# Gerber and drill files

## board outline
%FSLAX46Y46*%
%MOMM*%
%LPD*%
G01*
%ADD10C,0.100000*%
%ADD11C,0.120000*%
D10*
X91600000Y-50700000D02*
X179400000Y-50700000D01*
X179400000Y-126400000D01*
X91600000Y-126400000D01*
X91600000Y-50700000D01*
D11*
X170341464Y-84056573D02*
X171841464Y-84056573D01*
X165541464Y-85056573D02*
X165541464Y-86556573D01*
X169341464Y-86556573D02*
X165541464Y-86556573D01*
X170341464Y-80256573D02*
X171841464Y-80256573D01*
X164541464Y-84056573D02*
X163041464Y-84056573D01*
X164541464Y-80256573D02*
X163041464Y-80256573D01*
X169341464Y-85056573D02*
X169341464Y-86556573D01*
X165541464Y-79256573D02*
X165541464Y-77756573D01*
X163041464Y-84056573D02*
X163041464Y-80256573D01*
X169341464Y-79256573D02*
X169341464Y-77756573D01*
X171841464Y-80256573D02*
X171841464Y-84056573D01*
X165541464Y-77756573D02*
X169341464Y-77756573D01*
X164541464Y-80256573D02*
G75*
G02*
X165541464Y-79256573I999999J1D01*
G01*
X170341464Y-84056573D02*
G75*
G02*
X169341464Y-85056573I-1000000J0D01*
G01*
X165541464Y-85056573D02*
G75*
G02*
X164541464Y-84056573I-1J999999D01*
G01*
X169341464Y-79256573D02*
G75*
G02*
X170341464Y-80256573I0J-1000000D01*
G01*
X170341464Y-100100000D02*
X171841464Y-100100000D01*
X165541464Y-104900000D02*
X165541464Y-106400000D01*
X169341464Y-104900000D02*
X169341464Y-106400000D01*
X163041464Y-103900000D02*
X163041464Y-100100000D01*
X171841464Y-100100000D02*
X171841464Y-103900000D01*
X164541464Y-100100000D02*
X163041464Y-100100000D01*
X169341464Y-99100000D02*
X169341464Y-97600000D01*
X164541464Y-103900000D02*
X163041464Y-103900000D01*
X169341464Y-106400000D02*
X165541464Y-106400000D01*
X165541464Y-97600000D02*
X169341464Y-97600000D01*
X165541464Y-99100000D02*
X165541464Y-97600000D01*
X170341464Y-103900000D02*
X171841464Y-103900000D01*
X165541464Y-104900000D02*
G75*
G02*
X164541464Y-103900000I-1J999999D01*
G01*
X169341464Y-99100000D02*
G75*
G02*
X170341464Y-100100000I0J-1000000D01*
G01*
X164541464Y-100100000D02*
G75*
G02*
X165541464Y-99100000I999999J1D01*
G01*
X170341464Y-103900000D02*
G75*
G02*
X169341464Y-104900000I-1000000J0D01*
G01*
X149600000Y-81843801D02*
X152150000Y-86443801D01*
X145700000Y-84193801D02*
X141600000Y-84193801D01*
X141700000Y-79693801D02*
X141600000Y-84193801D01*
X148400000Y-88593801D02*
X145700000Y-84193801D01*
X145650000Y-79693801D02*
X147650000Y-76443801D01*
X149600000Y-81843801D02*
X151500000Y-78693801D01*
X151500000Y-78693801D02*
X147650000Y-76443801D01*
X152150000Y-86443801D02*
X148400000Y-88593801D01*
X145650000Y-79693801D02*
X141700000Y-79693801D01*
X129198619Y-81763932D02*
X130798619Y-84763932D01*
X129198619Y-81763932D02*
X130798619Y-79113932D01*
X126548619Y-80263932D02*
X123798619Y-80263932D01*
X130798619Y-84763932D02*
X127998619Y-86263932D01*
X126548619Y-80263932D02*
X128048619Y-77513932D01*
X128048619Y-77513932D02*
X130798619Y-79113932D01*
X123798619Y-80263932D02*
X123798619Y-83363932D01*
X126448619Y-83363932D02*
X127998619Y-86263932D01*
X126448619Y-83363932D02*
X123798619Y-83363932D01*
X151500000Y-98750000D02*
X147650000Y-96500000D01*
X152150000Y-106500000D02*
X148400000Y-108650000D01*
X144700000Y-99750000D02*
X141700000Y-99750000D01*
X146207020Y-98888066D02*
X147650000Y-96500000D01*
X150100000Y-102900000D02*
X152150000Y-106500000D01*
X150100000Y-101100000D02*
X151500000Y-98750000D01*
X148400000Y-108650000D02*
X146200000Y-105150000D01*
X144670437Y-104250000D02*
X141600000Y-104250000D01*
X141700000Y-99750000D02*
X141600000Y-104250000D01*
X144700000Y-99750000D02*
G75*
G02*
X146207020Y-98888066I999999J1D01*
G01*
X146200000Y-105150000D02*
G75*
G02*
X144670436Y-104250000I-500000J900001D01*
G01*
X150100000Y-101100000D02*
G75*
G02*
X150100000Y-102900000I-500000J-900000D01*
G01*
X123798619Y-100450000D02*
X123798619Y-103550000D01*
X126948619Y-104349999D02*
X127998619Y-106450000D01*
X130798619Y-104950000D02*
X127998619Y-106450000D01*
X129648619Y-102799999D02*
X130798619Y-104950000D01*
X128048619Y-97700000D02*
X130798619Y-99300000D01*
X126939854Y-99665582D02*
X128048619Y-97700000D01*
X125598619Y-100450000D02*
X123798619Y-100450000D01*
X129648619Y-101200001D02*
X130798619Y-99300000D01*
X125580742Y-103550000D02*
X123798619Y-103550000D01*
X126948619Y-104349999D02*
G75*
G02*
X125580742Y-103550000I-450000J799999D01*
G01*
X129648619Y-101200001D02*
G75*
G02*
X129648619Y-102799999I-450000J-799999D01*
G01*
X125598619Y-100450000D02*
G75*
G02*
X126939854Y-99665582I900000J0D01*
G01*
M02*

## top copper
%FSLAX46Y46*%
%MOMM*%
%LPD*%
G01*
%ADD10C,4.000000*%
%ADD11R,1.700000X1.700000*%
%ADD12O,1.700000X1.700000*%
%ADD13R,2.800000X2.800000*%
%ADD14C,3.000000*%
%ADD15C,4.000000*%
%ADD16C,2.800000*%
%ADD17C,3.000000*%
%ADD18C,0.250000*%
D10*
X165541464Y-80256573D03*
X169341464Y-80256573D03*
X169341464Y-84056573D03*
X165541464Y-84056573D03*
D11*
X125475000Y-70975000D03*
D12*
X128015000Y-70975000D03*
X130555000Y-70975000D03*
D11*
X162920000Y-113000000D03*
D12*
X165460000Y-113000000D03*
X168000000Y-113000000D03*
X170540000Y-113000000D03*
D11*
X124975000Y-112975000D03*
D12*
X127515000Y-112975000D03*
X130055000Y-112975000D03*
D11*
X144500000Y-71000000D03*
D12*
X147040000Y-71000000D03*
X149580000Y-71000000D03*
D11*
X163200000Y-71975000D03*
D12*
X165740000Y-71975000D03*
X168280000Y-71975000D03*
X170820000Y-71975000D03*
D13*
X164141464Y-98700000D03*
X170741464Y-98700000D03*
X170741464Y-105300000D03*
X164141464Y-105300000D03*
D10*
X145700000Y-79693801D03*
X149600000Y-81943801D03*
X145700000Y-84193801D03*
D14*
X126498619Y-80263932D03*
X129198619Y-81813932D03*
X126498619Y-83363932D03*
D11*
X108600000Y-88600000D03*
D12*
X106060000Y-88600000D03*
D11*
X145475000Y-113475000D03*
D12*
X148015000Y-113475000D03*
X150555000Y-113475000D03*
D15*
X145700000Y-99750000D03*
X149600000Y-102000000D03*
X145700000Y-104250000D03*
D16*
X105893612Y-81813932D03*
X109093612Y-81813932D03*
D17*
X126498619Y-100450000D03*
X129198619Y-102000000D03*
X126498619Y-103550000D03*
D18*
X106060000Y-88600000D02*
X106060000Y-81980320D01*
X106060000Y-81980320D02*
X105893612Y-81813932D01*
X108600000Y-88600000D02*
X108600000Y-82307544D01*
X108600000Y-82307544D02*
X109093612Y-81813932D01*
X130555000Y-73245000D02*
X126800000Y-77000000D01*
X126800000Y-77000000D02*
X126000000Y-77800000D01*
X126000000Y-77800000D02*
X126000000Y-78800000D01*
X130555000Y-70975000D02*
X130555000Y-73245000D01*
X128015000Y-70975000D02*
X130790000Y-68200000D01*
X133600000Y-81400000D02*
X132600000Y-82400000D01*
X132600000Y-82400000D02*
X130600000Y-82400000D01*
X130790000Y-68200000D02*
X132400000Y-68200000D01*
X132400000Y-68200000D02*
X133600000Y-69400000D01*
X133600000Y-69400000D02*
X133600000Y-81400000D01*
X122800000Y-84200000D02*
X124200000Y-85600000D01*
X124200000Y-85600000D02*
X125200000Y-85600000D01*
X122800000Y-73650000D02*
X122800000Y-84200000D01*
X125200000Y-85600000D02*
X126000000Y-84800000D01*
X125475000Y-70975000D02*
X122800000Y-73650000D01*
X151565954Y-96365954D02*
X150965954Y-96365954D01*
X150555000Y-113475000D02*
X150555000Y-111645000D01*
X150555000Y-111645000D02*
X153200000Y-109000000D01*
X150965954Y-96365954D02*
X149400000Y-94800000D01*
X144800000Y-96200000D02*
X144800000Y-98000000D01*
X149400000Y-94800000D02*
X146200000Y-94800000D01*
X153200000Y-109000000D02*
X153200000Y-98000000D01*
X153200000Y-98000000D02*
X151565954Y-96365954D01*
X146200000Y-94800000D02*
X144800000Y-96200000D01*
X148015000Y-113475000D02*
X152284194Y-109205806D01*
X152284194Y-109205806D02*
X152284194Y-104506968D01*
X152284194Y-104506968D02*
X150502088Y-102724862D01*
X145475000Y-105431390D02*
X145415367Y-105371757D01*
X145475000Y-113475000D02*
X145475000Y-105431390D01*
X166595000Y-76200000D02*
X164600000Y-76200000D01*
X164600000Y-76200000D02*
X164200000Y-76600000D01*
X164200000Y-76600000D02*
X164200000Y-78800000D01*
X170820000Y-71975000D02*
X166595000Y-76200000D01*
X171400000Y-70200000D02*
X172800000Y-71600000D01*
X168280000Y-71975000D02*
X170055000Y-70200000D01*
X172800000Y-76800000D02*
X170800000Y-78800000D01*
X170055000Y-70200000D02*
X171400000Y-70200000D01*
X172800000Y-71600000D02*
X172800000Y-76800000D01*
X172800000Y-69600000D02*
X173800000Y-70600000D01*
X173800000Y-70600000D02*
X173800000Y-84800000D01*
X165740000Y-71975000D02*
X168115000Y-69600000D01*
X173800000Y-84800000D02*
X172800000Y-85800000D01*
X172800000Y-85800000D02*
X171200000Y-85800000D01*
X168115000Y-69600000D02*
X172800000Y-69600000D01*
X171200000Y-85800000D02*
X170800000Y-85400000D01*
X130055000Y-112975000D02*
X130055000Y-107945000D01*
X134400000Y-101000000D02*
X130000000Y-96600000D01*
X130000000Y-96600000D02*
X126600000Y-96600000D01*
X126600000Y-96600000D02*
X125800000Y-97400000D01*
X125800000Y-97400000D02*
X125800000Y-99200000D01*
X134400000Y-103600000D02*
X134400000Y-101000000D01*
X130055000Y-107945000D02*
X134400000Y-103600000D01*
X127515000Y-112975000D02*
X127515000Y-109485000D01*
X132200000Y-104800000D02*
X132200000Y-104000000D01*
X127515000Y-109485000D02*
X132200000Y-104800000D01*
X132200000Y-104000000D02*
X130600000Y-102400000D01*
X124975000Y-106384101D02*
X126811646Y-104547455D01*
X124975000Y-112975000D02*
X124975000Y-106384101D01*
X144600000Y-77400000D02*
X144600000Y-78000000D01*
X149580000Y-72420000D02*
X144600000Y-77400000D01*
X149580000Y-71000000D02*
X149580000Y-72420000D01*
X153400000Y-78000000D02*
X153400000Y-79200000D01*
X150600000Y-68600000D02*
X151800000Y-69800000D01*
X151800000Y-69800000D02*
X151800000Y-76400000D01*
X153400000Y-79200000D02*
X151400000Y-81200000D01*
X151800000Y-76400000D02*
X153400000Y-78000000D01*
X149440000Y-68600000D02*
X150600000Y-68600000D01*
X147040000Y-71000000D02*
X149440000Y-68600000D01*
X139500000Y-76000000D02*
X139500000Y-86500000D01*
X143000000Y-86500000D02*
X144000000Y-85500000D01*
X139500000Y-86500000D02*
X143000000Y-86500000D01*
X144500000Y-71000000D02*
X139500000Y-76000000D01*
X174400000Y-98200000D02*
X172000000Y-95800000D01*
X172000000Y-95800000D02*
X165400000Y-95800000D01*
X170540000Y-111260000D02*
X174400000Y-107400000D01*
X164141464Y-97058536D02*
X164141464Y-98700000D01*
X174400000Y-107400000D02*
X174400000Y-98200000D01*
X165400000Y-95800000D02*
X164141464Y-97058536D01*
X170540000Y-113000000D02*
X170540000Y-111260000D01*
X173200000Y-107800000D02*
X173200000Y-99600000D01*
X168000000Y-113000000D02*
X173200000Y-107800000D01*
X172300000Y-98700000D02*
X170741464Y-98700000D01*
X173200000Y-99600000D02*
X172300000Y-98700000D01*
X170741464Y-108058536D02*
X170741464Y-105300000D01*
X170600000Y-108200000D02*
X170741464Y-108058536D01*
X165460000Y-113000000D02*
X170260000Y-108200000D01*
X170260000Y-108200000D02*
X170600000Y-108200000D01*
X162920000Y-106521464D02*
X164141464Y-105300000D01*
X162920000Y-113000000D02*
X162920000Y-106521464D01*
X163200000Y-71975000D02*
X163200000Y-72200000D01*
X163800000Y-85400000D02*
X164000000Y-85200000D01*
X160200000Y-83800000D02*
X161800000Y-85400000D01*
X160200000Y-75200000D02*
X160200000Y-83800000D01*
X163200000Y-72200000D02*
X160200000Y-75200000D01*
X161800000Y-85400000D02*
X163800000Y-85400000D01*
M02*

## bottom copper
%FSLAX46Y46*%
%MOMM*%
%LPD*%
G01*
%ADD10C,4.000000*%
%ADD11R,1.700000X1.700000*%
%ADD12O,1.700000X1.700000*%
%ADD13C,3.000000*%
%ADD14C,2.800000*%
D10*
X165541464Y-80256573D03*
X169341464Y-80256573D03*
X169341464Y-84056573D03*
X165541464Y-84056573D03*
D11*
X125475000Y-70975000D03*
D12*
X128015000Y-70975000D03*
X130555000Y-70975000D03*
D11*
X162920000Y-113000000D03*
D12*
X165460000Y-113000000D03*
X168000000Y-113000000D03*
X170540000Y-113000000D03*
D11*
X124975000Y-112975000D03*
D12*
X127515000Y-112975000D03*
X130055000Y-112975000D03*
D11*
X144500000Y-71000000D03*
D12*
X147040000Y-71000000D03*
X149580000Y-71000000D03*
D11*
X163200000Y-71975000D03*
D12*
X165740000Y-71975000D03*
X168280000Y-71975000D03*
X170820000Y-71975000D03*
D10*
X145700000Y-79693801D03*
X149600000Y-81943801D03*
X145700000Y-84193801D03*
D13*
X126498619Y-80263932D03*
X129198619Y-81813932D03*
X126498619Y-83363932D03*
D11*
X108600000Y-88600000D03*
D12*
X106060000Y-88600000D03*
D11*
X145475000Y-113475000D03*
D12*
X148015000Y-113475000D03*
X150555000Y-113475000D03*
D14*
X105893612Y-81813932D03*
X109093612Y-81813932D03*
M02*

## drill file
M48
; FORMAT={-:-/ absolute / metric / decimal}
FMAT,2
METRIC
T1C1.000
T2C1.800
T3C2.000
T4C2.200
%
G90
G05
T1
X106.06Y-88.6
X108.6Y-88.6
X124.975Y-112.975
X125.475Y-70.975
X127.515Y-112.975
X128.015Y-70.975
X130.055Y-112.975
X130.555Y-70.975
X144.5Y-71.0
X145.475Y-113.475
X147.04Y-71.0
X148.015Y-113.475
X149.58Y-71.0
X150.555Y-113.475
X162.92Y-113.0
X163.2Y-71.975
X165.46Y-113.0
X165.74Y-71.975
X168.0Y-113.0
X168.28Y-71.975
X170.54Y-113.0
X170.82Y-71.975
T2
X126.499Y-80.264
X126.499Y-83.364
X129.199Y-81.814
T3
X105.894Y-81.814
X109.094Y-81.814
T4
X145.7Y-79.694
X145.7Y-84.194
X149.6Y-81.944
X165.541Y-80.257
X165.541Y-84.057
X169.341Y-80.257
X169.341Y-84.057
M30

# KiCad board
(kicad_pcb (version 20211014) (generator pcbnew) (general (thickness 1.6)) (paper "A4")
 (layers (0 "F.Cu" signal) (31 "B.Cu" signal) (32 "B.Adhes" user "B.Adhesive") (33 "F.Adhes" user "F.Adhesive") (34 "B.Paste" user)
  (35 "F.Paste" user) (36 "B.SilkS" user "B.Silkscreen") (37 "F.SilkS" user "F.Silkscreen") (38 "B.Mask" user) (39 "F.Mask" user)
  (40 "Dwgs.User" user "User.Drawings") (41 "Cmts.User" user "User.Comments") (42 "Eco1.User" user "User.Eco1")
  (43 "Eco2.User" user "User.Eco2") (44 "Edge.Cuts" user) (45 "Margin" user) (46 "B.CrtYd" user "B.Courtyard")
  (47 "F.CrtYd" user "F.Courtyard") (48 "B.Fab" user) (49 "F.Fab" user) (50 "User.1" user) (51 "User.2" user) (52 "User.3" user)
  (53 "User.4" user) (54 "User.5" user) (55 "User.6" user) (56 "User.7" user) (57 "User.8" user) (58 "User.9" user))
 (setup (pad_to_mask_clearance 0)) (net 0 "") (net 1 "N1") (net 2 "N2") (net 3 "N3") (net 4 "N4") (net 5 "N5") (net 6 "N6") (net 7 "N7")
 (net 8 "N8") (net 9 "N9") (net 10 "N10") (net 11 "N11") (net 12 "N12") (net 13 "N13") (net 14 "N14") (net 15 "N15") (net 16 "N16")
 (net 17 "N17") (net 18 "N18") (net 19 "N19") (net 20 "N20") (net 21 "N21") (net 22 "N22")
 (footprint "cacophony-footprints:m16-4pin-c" (layer "F.Cu") (at 167.441464 82.156573)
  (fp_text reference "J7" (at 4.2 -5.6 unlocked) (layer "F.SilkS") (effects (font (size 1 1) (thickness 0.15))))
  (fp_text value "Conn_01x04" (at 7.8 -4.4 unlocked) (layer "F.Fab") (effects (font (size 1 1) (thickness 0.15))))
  (fp_line (start 2.9 1.9) (end 4.4 1.9) (layer "Edge.Cuts") (width 0.12))
  (fp_line (start -1.9 2.9) (end -1.9 4.4) (layer "Edge.Cuts") (width 0.12))
  (fp_line (start 1.9 4.4) (end -1.9 4.4) (layer "Edge.Cuts") (width 0.12))
  (fp_line (start 2.9 -1.9) (end 4.4 -1.9) (layer "Edge.Cuts") (width 0.12))
  (fp_line (start -2.9 1.9) (end -4.4 1.9) (layer "Edge.Cuts") (width 0.12))
  (fp_line (start -2.9 -1.9) (end -4.4 -1.9) (layer "Edge.Cuts") (width 0.12))
  (fp_line (start 1.9 2.9) (end 1.9 4.4) (layer "Edge.Cuts") (width 0.12))
  (fp_line (start -1.9 -2.9) (end -1.9 -4.4) (layer "Edge.Cuts") (width 0.12))
  (fp_line (start -4.4 1.9) (end -4.4 -1.9) (layer "Edge.Cuts") (width 0.12))
  (fp_line (start 1.9 -2.9) (end 1.9 -4.4) (layer "Edge.Cuts") (width 0.12))
  (fp_line (start 4.4 -1.9) (end 4.4 1.9) (layer "Edge.Cuts") (width 0.12))
  (fp_line (start -1.9 -4.4) (end 1.9 -4.4) (layer "Edge.Cuts") (width 0.12))
  (fp_arc (start -2.9 -1.9) (mid -2.607107 -2.607107) (end -1.9 -2.9) (layer "Edge.Cuts") (width 0.12))
  (fp_arc (start 2.9 1.9) (mid 2.607107 2.607107) (end 1.9 2.9) (layer "Edge.Cuts") (width 0.12))
  (fp_arc (start -1.9 2.9) (mid -2.607107 2.607107) (end -2.9 1.9) (layer "Edge.Cuts") (width 0.12))
  (fp_arc (start 1.9 -2.9) (mid 2.607107 -2.607107) (end 2.9 -1.9) (layer "Edge.Cuts") (width 0.12))
  (pad "1" thru_hole circle (at -1.9 -1.9) (size 4 4) (drill 2.2) (layers *.Cu *.Mask) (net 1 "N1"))
  (pad "2" thru_hole circle (at 1.9 -1.9) (size 4 4) (drill 2.2) (layers *.Cu *.Mask) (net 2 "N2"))
  (pad "3" thru_hole circle (at 1.9 1.9) (size 4 4) (drill 2.2) (layers *.Cu *.Mask) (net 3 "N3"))
  (pad "4" thru_hole circle (at -1.9 1.9) (size 4 4) (drill 2.2) (layers *.Cu *.Mask) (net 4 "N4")))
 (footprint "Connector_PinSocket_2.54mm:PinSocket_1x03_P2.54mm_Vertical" (layer "F.Cu") (at 125.475 70.975 90)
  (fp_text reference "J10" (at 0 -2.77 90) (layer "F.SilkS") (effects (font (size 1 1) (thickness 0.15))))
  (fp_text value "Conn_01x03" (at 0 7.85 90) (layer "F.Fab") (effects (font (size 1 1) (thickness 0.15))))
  (pad "1" thru_hole rect (at 0 0 90) (size 1.7 1.7) (drill 1) (layers *.Cu *.Mask) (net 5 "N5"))
  (pad "2" thru_hole oval (at 0 2.54 90) (size 1.7 1.7) (drill 1) (layers *.Cu *.Mask) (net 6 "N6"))
  (pad "3" thru_hole oval (at 0 5.08 90) (size 1.7 1.7) (drill 1) (layers *.Cu *.Mask) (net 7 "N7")))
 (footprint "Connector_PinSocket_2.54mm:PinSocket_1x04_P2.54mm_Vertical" (layer "F.Cu") (at 162.92 113 90)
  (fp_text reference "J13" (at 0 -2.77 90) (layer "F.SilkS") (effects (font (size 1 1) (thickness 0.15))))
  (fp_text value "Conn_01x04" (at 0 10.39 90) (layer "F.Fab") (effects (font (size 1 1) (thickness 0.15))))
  (pad "1" thru_hole rect (at 0 0 90) (size 1.7 1.7) (drill 1) (layers *.Cu *.Mask) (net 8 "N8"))
  (pad "2" thru_hole oval (at 0 2.54 90) (size 1.7 1.7) (drill 1) (layers *.Cu *.Mask) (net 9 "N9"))
  (pad "3" thru_hole oval (at 0 5.08 90) (size 1.7 1.7) (drill 1) (layers *.Cu *.Mask) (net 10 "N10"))
  (pad "4" thru_hole oval (at 0 7.62 90) (size 1.7 1.7) (drill 1) (layers *.Cu *.Mask) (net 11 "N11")))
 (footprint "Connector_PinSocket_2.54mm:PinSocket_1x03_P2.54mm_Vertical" (layer "F.Cu") (at 124.975 112.975 90)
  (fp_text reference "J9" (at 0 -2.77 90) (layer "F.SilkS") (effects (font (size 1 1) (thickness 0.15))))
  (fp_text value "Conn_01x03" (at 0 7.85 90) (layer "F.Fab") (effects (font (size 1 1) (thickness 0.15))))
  (pad "1" thru_hole rect (at 0 0 90) (size 1.7 1.7) (drill 1) (layers *.Cu *.Mask) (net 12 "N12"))
  (pad "2" thru_hole oval (at 0 2.54 90) (size 1.7 1.7) (drill 1) (layers *.Cu *.Mask) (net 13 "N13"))
  (pad "3" thru_hole oval (at 0 5.08 90) (size 1.7 1.7) (drill 1) (layers *.Cu *.Mask) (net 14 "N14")))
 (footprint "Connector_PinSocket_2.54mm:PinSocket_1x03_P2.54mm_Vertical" (layer "F.Cu") (at 144.5 71 90)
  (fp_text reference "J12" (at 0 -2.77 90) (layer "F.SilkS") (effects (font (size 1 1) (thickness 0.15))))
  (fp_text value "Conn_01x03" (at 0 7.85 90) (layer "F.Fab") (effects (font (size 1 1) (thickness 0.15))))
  (pad "1" thru_hole rect (at 0 0 90) (size 1.7 1.7) (drill 1) (layers *.Cu *.Mask) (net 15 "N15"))
  (pad "2" thru_hole oval (at 0 2.54 90) (size 1.7 1.7) (drill 1) (layers *.Cu *.Mask) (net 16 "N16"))
  (pad "3" thru_hole oval (at 0 5.08 90) (size 1.7 1.7) (drill 1) (layers *.Cu *.Mask) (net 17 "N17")))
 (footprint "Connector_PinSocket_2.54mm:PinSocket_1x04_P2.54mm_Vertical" (layer "F.Cu") (at 163.2 71.975 90)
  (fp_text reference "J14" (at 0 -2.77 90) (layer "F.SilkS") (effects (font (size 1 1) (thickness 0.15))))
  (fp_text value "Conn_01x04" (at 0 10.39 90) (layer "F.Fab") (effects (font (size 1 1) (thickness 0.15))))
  (pad "1" thru_hole rect (at 0 0 90) (size 1.7 1.7) (drill 1) (layers *.Cu *.Mask) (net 4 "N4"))
  (pad "2" thru_hole oval (at 0 2.54 90) (size 1.7 1.7) (drill 1) (layers *.Cu *.Mask) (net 3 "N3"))
  (pad "3" thru_hole oval (at 0 5.08 90) (size 1.7 1.7) (drill 1) (layers *.Cu *.Mask) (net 2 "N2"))
  (pad "4" thru_hole oval (at 0 7.62 90) (size 1.7 1.7) (drill 1) (layers *.Cu *.Mask) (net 1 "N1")))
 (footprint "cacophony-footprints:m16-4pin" (layer "F.Cu") (at 167.441464 102)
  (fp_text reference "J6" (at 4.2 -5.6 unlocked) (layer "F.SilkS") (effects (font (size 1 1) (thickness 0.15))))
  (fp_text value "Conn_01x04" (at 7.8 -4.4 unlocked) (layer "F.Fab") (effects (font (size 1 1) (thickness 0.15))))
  (fp_line (start 2.9 -1.9) (end 4.4 -1.9) (layer "Edge.Cuts") (width 0.12))
  (fp_line (start -1.9 2.9) (end -1.9 4.4) (layer "Edge.Cuts") (width 0.12))
  (fp_line (start 1.9 2.9) (end 1.9 4.4) (layer "Edge.Cuts") (width 0.12))
  (fp_line (start -4.4 1.9) (end -4.4 -1.9) (layer "Edge.Cuts") (width 0.12))
  (fp_line (start 4.4 -1.9) (end 4.4 1.9) (layer "Edge.Cuts") (width 0.12))
  (fp_line (start -2.9 -1.9) (end -4.4 -1.9) (layer "Edge.Cuts") (width 0.12))
  (fp_line (start 1.9 -2.9) (end 1.9 -4.4) (layer "Edge.Cuts") (width 0.12))
  (fp_line (start -2.9 1.9) (end -4.4 1.9) (layer "Edge.Cuts") (width 0.12))
  (fp_line (start 1.9 4.4) (end -1.9 4.4) (layer "Edge.Cuts") (width 0.12))
  (fp_line (start -1.9 -4.4) (end 1.9 -4.4) (layer "Edge.Cuts") (width 0.12))
  (fp_line (start -1.9 -2.9) (end -1.9 -4.4) (layer "Edge.Cuts") (width 0.12))
  (fp_line (start 2.9 1.9) (end 4.4 1.9) (layer "Edge.Cuts") (width 0.12))
  (fp_arc (start -1.9 2.9) (mid -2.607107 2.607107) (end -2.9 1.9) (layer "Edge.Cuts") (width 0.12))
  (fp_arc (start 1.9 -2.9) (mid 2.607107 -2.607107) (end 2.9 -1.9) (layer "Edge.Cuts") (width 0.12))
  (fp_arc (start -2.9 -1.9) (mid -2.607107 -2.607107) (end -1.9 -2.9) (layer "Edge.Cuts") (width 0.12))
  (fp_arc (start 2.9 1.9) (mid 2.607107 2.607107) (end 1.9 2.9) (layer "Edge.Cuts") (width 0.12))
  (pad "1" smd rect (at -3.3 -3.3) (size 2.8 2.8) (layers "F.Cu" "F.Paste" "F.Mask") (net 11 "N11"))
  (pad "2" smd rect (at 3.3 -3.3) (size 2.8 2.8) (layers "F.Cu" "F.Paste" "F.Mask") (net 10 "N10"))
  (pad "3" smd rect (at 3.3 3.3) (size 2.8 2.8) (layers "F.Cu" "F.Paste" "F.Mask") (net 9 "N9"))
  (pad "4" smd rect (at -3.3 3.3) (size 2.8 2.8) (layers "F.Cu" "F.Paste" "F.Mask") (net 8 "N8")))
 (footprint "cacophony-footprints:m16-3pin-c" (layer "F.Cu") (at 147 81.943801)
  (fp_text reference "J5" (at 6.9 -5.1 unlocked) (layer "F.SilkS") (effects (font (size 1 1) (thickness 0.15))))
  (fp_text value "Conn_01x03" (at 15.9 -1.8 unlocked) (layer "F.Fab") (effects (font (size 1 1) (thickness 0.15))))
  (fp_line (start 2.6 -0.1) (end 5.15 4.5) (layer "Edge.Cuts") (width 0.12))
  (fp_line (start -1.3 2.25) (end -5.4 2.25) (layer "Edge.Cuts") (width 0.12))
  (fp_line (start -5.3 -2.25) (end -5.4 2.25) (layer "Edge.Cuts") (width 0.12))
  (fp_line (start 1.4 6.65) (end -1.3 2.25) (layer "Edge.Cuts") (width 0.12))
  (fp_line (start -1.35 -2.25) (end 0.65 -5.5) (layer "Edge.Cuts") (width 0.12))
  (fp_line (start 2.6 -0.1) (end 4.5 -3.25) (layer "Edge.Cuts") (width 0.12))
  (fp_line (start 4.5 -3.25) (end 0.65 -5.5) (layer "Edge.Cuts") (width 0.12))
  (fp_line (start 5.15 4.5) (end 1.4 6.65) (layer "Edge.Cuts") (width 0.12))
  (fp_line (start -1.35 -2.25) (end -5.3 -2.25) (layer "Edge.Cuts") (width 0.12))
  (pad "1" thru_hole circle (at -1.3 -2.25) (size 4 4) (drill 2.2) (layers *.Cu *.Mask) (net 17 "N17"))
  (pad "2" thru_hole circle (at 2.6 0) (size 4 4) (drill 2.2) (layers *.Cu *.Mask) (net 16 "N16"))
  (pad "3" thru_hole circle (at -1.3 2.25) (size 4 4) (drill 2.2) (layers *.Cu *.Mask) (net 15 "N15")))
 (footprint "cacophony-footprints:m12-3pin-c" (layer "F.Cu") (at 127.398619 81.813932)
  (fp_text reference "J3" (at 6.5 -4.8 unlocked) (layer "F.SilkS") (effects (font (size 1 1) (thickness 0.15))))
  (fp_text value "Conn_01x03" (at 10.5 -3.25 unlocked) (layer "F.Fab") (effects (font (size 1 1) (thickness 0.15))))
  (fp_line (start 1.8 -0.05) (end 3.4 2.95) (layer "Edge.Cuts") (width 0.12))
  (fp_line (start 1.8 -0.05) (end 3.4 -2.7) (layer "Edge.Cuts") (width 0.12))
  (fp_line (start -0.85 -1.55) (end -3.6 -1.55) (layer "Edge.Cuts") (width 0.12))
  (fp_line (start 3.4 2.95) (end 0.6 4.45) (layer "Edge.Cuts") (width 0.12))
  (fp_line (start -0.85 -1.55) (end 0.65 -4.3) (layer "Edge.Cuts") (width 0.12))
  (fp_line (start 0.65 -4.3) (end 3.4 -2.7) (layer "Edge.Cuts") (width 0.12))
  (fp_line (start -3.6 -1.55) (end -3.6 1.55) (layer "Edge.Cuts") (width 0.12))
  (fp_line (start -0.95 1.55) (end 0.6 4.45) (layer "Edge.Cuts") (width 0.12))
  (fp_line (start -0.95 1.55) (end -3.6 1.55) (layer "Edge.Cuts") (width 0.12))
  (pad "1" thru_hole circle (at -0.9 -1.55) (size 3 3) (drill 1.8) (layers *.Cu *.Mask) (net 7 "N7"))
  (pad "2" thru_hole circle (at 1.8 0) (size 3 3) (drill 1.8) (layers *.Cu *.Mask) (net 6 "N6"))
  (pad "3" thru_hole circle (at -0.9 1.55) (size 3 3) (drill 1.8) (layers *.Cu *.Mask) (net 5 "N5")))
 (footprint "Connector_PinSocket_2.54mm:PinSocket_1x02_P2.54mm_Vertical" (layer "F.Cu") (at 108.6 88.6 -90)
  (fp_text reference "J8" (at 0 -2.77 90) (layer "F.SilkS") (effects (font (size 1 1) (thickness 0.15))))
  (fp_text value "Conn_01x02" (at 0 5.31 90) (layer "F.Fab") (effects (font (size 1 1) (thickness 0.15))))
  (pad "1" thru_hole rect (at 0 0 270) (size 1.7 1.7) (drill 1) (layers *.Cu *.Mask) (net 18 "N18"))
  (pad "2" thru_hole oval (at 0 2.54 270) (size 1.7 1.7) (drill 1) (layers *.Cu *.Mask) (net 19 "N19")))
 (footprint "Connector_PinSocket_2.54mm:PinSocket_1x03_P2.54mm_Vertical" (layer "F.Cu") (at 145.475 113.475 90)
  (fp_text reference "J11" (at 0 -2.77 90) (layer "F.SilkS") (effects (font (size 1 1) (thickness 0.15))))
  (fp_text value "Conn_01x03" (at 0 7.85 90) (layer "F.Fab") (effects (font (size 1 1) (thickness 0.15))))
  (pad "1" thru_hole rect (at 0 0 90) (size 1.7 1.7) (drill 1) (layers *.Cu *.Mask) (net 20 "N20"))
  (pad "2" thru_hole oval (at 0 2.54 90) (size 1.7 1.7) (drill 1) (layers *.Cu *.Mask) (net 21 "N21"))
  (pad "3" thru_hole oval (at 0 5.08 90) (size 1.7 1.7) (drill 1) (layers *.Cu *.Mask) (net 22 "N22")))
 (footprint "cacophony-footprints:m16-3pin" (layer "F.Cu") (at 147 102)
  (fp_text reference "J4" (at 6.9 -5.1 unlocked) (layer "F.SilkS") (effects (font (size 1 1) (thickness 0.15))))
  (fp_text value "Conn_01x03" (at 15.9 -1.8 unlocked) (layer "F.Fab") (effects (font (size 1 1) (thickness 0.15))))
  (fp_line (start 4.5 -3.25) (end 0.65 -5.5) (layer "Edge.Cuts") (width 0.12))
  (fp_line (start 5.15 4.5) (end 1.4 6.65) (layer "Edge.Cuts") (width 0.12))
  (fp_line (start -2.3 -2.25) (end -5.3 -2.25) (layer "Edge.Cuts") (width 0.12))
  (fp_line (start -0.79298 -3.111934) (end 0.65 -5.5) (layer "Edge.Cuts") (width 0.12))
  (fp_line (start 3.1 0.9) (end 5.15 4.5) (layer "Edge.Cuts") (width 0.12))
  (fp_line (start 3.1 -0.9) (end 4.5 -3.25) (layer "Edge.Cuts") (width 0.12))
  (fp_line (start 1.4 6.65) (end -0.8 3.15) (layer "Edge.Cuts") (width 0.12))
  (fp_line (start -2.329563 2.25) (end -5.4 2.25) (layer "Edge.Cuts") (width 0.12))
  (fp_line (start -5.3 -2.25) (end -5.4 2.25) (layer "Edge.Cuts") (width 0.12))
  (fp_arc (start -2.3 -2.25) (mid -1.796478 -3.11805) (end -0.79298 -3.111934) (layer "Edge.Cuts") (width 0.12))
  (fp_arc (start -0.8 3.15) (mid -1.82212 3.13735) (end -2.329563 2.25) (layer "Edge.Cuts") (width 0.12))
  (fp_arc (start 3.1 -0.9) (mid 3.629563 0) (end 3.1 0.9) (layer "Edge.Cuts") (width 0.12))
  (pad "1" smd circle (at -1.3 -2.25) (size 4 4) (layers "F.Cu" "F.Paste" "F.Mask") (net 22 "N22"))
  (pad "2" smd circle (at 2.6 0) (size 4 4) (layers "F.Cu" "F.Paste" "F.Mask") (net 21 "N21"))
  (pad "3" smd circle (at -1.3 2.25) (size 4 4) (layers "F.Cu" "F.Paste" "F.Mask") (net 20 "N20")))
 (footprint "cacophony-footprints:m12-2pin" (layer "F.Cu") (at 107.493612 81.813932)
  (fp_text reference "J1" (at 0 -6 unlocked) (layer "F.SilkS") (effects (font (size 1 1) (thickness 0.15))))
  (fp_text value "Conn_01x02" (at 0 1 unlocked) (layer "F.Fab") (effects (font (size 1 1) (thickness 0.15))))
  (pad "1" thru_hole circle (at -1.6 0) (size 2.8 2.8) (drill 2) (layers *.Cu *.Mask) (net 19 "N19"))
  (pad "2" thru_hole circle (at 1.6 0) (size 2.8 2.8) (drill 2) (layers *.Cu *.Mask) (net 18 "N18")))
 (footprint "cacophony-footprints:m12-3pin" (layer "F.Cu") (at 127.398619 102)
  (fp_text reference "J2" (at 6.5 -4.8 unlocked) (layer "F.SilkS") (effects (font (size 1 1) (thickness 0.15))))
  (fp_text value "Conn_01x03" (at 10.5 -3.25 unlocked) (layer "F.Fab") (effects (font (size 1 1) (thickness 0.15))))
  (fp_line (start -3.6 -1.55) (end -3.6 1.55) (layer "Edge.Cuts") (width 0.12))
  (fp_line (start -0.45 2.349999) (end 0.6 4.45) (layer "Edge.Cuts") (width 0.12))
  (fp_line (start 3.4 2.95) (end 0.6 4.45) (layer "Edge.Cuts") (width 0.12))
  (fp_line (start 2.25 0.799999) (end 3.4 2.95) (layer "Edge.Cuts") (width 0.12))
  (fp_line (start 0.65 -4.3) (end 3.4 -2.7) (layer "Edge.Cuts") (width 0.12))
  (fp_line (start -0.458765 -2.334418) (end 0.65 -4.3) (layer "Edge.Cuts") (width 0.12))
  (fp_line (start -1.8 -1.55) (end -3.6 -1.55) (layer "Edge.Cuts") (width 0.12))
  (fp_line (start 2.25 -0.799999) (end 3.4 -2.7) (layer "Edge.Cuts") (width 0.12))
  (fp_line (start -1.817877 1.55) (end -3.6 1.55) (layer "Edge.Cuts") (width 0.12))
  (fp_arc (start -0.45 2.349999) (mid -1.363387 2.34232) (end -1.817877 1.55) (layer "Edge.Cuts") (width 0.12))
  (fp_arc (start 2.25 -0.799999) (mid 2.717877 0) (end 2.25 0.799999) (layer "Edge.Cuts") (width 0.12))
  (fp_arc (start -1.8 -1.55) (mid -1.354361 -2.326889) (end -0.458765 -2.334418) (layer "Edge.Cuts") (width 0.12))
  (pad "1" smd circle (at -0.9 -1.55) (size 3 3) (layers "F.Cu" "F.Paste" "F.Mask") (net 14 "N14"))
  (pad "2" smd circle (at 1.8 0) (size 3 3) (layers "F.Cu" "F.Paste" "F.Mask") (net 13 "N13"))
  (pad "3" smd circle (at -0.9 1.55) (size 3 3) (layers "F.Cu" "F.Paste" "F.Mask") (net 12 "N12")))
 (gr_rect (start 91.6 50.7) (end 179.4 126.4) (layer "Edge.Cuts") (width 0.1) (fill none))
 (segment (start 106.06 88.6) (end 106.06 81.98032) (width 0.25) (layer "F.Cu") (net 19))
 (segment (start 106.06 81.98032) (end 105.893612 81.813932) (width 0.25) (layer "F.Cu") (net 19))
 (segment (start 108.6 88.6) (end 108.6 82.307544) (width 0.25) (layer "F.Cu") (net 18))
 (segment (start 108.6 82.307544) (end 109.093612 81.813932) (width 0.25) (layer "F.Cu") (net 18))
 (segment (start 130.555 73.245) (end 126.8 77) (width 0.25) (layer "F.Cu") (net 7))
 (segment (start 126.8 77) (end 126 77.8) (width 0.25) (layer "F.Cu") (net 7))
 (segment (start 126 77.8) (end 126 78.8) (width 0.25) (layer "F.Cu") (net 7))
 (segment (start 130.555 70.975) (end 130.555 73.245) (width 0.25) (layer "F.Cu") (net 7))
 (segment (start 128.015 70.975) (end 130.79 68.2) (width 0.25) (layer "F.Cu") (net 6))
 (segment (start 133.6 81.4) (end 132.6 82.4) (width 0.25) (layer "F.Cu") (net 6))
 (segment (start 132.6 82.4) (end 130.6 82.4) (width 0.25) (layer "F.Cu") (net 6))
 (segment (start 130.79 68.2) (end 132.4 68.2) (width 0.25) (layer "F.Cu") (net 6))
 (segment (start 132.4 68.2) (end 133.6 69.4) (width 0.25) (layer "F.Cu") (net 6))
 (segment (start 133.6 69.4) (end 133.6 81.4) (width 0.25) (layer "F.Cu") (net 6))
 (segment (start 122.8 84.2) (end 124.2 85.6) (width 0.25) (layer "F.Cu") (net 5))
 (segment (start 124.2 85.6) (end 125.2 85.6) (width 0.25) (layer "F.Cu") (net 5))
 (segment (start 122.8 73.65) (end 122.8 84.2) (width 0.25) (layer "F.Cu") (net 5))
 (segment (start 125.2 85.6) (end 126 84.8) (width 0.25) (layer "F.Cu") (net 5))
 (segment (start 125.475 70.975) (end 122.8 73.65) (width 0.25) (layer "F.Cu") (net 5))
 (segment (start 151.565954 96.365954) (end 150.965954 96.365954) (width 0.25) (layer "F.Cu") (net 22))
 (segment (start 150.555 113.475) (end 150.555 111.645) (width 0.25) (layer "F.Cu") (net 22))
 (segment (start 150.555 111.645) (end 153.2 109) (width 0.25) (layer "F.Cu") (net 22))
 (segment (start 150.965954 96.365954) (end 149.4 94.8) (width 0.25) (layer "F.Cu") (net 22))
 (segment (start 144.8 96.2) (end 144.8 98) (width 0.25) (layer "F.Cu") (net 22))
 (segment (start 149.4 94.8) (end 146.2 94.8) (width 0.25) (layer "F.Cu") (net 22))
 (segment (start 153.2 109) (end 153.2 98) (width 0.25) (layer "F.Cu") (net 22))
 (segment (start 153.2 98) (end 151.565954 96.365954) (width 0.25) (layer "F.Cu") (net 22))
 (segment (start 146.2 94.8) (end 144.8 96.2) (width 0.25) (layer "F.Cu") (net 22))
 (segment (start 148.015 113.475) (end 152.284194 109.205806) (width 0.25) (layer "F.Cu") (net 21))
 (segment (start 152.284194 109.205806) (end 152.284194 104.506968) (width 0.25) (layer "F.Cu") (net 21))
 (segment (start 152.284194 104.506968) (end 150.502088 102.724862) (width 0.25) (layer "F.Cu") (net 21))
 (segment (start 145.475 105.43139) (end 145.415367 105.371757) (width 0.25) (layer "F.Cu") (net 20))
 (segment (start 145.475 113.475) (end 145.475 105.43139) (width 0.25) (layer "F.Cu") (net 20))
 (segment (start 166.595 76.2) (end 164.6 76.2) (width 0.25) (layer "F.Cu") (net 1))
 (segment (start 164.6 76.2) (end 164.2 76.6) (width 0.25) (layer "F.Cu") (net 1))
 (segment (start 164.2 76.6) (end 164.2 78.8) (width 0.25) (layer "F.Cu") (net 1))
 (segment (start 170.82 71.975) (end 166.595 76.2) (width 0.25) (layer "F.Cu") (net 1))
 (segment (start 171.4 70.2) (end 172.8 71.6) (width 0.25) (layer "F.Cu") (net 2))
 (segment (start 168.28 71.975) (end 170.055 70.2) (width 0.25) (layer "F.Cu") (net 2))
 (segment (start 172.8 76.8) (end 170.8 78.8) (width 0.25) (layer "F.Cu") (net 2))
 (segment (start 170.055 70.2) (end 171.4 70.2) (width 0.25) (layer "F.Cu") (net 2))
 (segment (start 172.8 71.6) (end 172.8 76.8) (width 0.25) (layer "F.Cu") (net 2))
 (segment (start 172.8 69.6) (end 173.8 70.6) (width 0.25) (layer "F.Cu") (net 3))
 (segment (start 173.8 70.6) (end 173.8 84.8) (width 0.25) (layer "F.Cu") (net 3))
 (segment (start 165.74 71.975) (end 168.115 69.6) (width 0.25) (layer "F.Cu") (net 3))
 (segment (start 173.8 84.8) (end 172.8 85.8) (width 0.25) (layer "F.Cu") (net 3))
 (segment (start 172.8 85.8) (end 171.2 85.8) (width 0.25) (layer "F.Cu") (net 3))
 (segment (start 168.115 69.6) (end 172.8 69.6) (width 0.25) (layer "F.Cu") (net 3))
 (segment (start 171.2 85.8) (end 170.8 85.4) (width 0.25) (layer "F.Cu") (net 3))
 (segment (start 130.055 112.975) (end 130.055 107.945) (width 0.25) (layer "F.Cu") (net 14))
 (segment (start 134.4 101) (end 130 96.6) (width 0.25) (layer "F.Cu") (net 14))
 (segment (start 130 96.6) (end 126.6 96.6) (width 0.25) (layer "F.Cu") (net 14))
 (segment (start 126.6 96.6) (end 125.8 97.4) (width 0.25) (layer "F.Cu") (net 14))
 (segment (start 125.8 97.4) (end 125.8 99.2) (width 0.25) (layer "F.Cu") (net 14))
 (segment (start 134.4 103.6) (end 134.4 101) (width 0.25) (layer "F.Cu") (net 14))
 (segment (start 130.055 107.945) (end 134.4 103.6) (width 0.25) (layer "F.Cu") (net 14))
 (segment (start 127.515 112.975) (end 127.515 109.485) (width 0.25) (layer "F.Cu") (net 13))
 (segment (start 132.2 104.8) (end 132.2 104) (width 0.25) (layer "F.Cu") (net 13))
 (segment (start 127.515 109.485) (end 132.2 104.8) (width 0.25) (layer "F.Cu") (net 13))
 (segment (start 132.2 104) (end 130.6 102.4) (width 0.25) (layer "F.Cu") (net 13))
 (segment (start 124.975 106.384101) (end 126.811646 104.547455) (width 0.25) (layer "F.Cu") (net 12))
 (segment (start 124.975 112.975) (end 124.975 106.384101) (width 0.25) (layer "F.Cu") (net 12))
 (segment (start 144.6 77.4) (end 144.6 78) (width 0.25) (layer "F.Cu") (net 17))
 (segment (start 149.58 72.42) (end 144.6 77.4) (width 0.25) (layer "F.Cu") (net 17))
 (segment (start 149.58 71) (end 149.58 72.42) (width 0.25) (layer "F.Cu") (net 17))
 (segment (start 153.4 78) (end 153.4 79.2) (width 0.25) (layer "F.Cu") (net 16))
 (segment (start 150.6 68.6) (end 151.8 69.8) (width 0.25) (layer "F.Cu") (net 16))
 (segment (start 151.8 69.8) (end 151.8 76.4) (width 0.25) (layer "F.Cu") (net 16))
 (segment (start 153.4 79.2) (end 151.4 81.2) (width 0.25) (layer "F.Cu") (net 16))
 (segment (start 151.8 76.4) (end 153.4 78) (width 0.25) (layer "F.Cu") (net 16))
 (segment (start 149.44 68.6) (end 150.6 68.6) (width 0.25) (layer "F.Cu") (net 16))
 (segment (start 147.04 71) (end 149.44 68.6) (width 0.25) (layer "F.Cu") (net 16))
 (segment (start 139.5 76) (end 139.5 86.5) (width 0.25) (layer "F.Cu") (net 15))
 (segment (start 143 86.5) (end 144 85.5) (width 0.25) (layer "F.Cu") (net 15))
 (segment (start 139.5 86.5) (end 143 86.5) (width 0.25) (layer "F.Cu") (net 15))
 (segment (start 144.5 71) (end 139.5 76) (width 0.25) (layer "F.Cu") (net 15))
 (segment (start 174.4 98.2) (end 172 95.8) (width 0.25) (layer "F.Cu") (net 11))
 (segment (start 172 95.8) (end 165.4 95.8) (width 0.25) (layer "F.Cu") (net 11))
 (segment (start 170.54 111.26) (end 174.4 107.4) (width 0.25) (layer "F.Cu") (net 11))
 (segment (start 164.141464 97.058536) (end 164.141464 98.7) (width 0.25) (layer "F.Cu") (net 11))
 (segment (start 174.4 107.4) (end 174.4 98.2) (width 0.25) (layer "F.Cu") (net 11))
 (segment (start 165.4 95.8) (end 164.141464 97.058536) (width 0.25) (layer "F.Cu") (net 11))
 (segment (start 170.54 113) (end 170.54 111.26) (width 0.25) (layer "F.Cu") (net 11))
 (segment (start 173.2 107.8) (end 173.2 99.6) (width 0.25) (layer "F.Cu") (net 10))
 (segment (start 168 113) (end 173.2 107.8) (width 0.25) (layer "F.Cu") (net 10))
 (segment (start 172.3 98.7) (end 170.741464 98.7) (width 0.25) (layer "F.Cu") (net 10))
 (segment (start 173.2 99.6) (end 172.3 98.7) (width 0.25) (layer "F.Cu") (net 10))
 (segment (start 170.741464 108.058536) (end 170.741464 105.3) (width 0.25) (layer "F.Cu") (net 9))
 (segment (start 170.6 108.2) (end 170.741464 108.058536) (width 0.25) (layer "F.Cu") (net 9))
 (segment (start 165.46 113) (end 170.26 108.2) (width 0.25) (layer "F.Cu") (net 9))
 (segment (start 170.26 108.2) (end 170.6 108.2) (width 0.25) (layer "F.Cu") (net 9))
 (segment (start 162.92 106.521464) (end 164.141464 105.3) (width 0.25) (layer "F.Cu") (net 8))
 (segment (start 162.92 113) (end 162.92 106.521464) (width 0.25) (layer "F.Cu") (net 8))
 (segment (start 163.2 71.975) (end 163.2 72.2) (width 0.25) (layer "F.Cu") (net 4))
 (segment (start 163.8 85.4) (end 164 85.2) (width 0.25) (layer "F.Cu") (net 4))
 (segment (start 160.2 83.8) (end 161.8 85.4) (width 0.25) (layer "F.Cu") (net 4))
 (segment (start 160.2 75.2) (end 160.2 83.8) (width 0.25) (layer "F.Cu") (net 4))
 (segment (start 163.2 72.2) (end 160.2 75.2) (width 0.25) (layer "F.Cu") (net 4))
 (segment (start 161.8 85.4) (end 163.8 85.4) (width 0.25) (layer "F.Cu") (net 4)))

